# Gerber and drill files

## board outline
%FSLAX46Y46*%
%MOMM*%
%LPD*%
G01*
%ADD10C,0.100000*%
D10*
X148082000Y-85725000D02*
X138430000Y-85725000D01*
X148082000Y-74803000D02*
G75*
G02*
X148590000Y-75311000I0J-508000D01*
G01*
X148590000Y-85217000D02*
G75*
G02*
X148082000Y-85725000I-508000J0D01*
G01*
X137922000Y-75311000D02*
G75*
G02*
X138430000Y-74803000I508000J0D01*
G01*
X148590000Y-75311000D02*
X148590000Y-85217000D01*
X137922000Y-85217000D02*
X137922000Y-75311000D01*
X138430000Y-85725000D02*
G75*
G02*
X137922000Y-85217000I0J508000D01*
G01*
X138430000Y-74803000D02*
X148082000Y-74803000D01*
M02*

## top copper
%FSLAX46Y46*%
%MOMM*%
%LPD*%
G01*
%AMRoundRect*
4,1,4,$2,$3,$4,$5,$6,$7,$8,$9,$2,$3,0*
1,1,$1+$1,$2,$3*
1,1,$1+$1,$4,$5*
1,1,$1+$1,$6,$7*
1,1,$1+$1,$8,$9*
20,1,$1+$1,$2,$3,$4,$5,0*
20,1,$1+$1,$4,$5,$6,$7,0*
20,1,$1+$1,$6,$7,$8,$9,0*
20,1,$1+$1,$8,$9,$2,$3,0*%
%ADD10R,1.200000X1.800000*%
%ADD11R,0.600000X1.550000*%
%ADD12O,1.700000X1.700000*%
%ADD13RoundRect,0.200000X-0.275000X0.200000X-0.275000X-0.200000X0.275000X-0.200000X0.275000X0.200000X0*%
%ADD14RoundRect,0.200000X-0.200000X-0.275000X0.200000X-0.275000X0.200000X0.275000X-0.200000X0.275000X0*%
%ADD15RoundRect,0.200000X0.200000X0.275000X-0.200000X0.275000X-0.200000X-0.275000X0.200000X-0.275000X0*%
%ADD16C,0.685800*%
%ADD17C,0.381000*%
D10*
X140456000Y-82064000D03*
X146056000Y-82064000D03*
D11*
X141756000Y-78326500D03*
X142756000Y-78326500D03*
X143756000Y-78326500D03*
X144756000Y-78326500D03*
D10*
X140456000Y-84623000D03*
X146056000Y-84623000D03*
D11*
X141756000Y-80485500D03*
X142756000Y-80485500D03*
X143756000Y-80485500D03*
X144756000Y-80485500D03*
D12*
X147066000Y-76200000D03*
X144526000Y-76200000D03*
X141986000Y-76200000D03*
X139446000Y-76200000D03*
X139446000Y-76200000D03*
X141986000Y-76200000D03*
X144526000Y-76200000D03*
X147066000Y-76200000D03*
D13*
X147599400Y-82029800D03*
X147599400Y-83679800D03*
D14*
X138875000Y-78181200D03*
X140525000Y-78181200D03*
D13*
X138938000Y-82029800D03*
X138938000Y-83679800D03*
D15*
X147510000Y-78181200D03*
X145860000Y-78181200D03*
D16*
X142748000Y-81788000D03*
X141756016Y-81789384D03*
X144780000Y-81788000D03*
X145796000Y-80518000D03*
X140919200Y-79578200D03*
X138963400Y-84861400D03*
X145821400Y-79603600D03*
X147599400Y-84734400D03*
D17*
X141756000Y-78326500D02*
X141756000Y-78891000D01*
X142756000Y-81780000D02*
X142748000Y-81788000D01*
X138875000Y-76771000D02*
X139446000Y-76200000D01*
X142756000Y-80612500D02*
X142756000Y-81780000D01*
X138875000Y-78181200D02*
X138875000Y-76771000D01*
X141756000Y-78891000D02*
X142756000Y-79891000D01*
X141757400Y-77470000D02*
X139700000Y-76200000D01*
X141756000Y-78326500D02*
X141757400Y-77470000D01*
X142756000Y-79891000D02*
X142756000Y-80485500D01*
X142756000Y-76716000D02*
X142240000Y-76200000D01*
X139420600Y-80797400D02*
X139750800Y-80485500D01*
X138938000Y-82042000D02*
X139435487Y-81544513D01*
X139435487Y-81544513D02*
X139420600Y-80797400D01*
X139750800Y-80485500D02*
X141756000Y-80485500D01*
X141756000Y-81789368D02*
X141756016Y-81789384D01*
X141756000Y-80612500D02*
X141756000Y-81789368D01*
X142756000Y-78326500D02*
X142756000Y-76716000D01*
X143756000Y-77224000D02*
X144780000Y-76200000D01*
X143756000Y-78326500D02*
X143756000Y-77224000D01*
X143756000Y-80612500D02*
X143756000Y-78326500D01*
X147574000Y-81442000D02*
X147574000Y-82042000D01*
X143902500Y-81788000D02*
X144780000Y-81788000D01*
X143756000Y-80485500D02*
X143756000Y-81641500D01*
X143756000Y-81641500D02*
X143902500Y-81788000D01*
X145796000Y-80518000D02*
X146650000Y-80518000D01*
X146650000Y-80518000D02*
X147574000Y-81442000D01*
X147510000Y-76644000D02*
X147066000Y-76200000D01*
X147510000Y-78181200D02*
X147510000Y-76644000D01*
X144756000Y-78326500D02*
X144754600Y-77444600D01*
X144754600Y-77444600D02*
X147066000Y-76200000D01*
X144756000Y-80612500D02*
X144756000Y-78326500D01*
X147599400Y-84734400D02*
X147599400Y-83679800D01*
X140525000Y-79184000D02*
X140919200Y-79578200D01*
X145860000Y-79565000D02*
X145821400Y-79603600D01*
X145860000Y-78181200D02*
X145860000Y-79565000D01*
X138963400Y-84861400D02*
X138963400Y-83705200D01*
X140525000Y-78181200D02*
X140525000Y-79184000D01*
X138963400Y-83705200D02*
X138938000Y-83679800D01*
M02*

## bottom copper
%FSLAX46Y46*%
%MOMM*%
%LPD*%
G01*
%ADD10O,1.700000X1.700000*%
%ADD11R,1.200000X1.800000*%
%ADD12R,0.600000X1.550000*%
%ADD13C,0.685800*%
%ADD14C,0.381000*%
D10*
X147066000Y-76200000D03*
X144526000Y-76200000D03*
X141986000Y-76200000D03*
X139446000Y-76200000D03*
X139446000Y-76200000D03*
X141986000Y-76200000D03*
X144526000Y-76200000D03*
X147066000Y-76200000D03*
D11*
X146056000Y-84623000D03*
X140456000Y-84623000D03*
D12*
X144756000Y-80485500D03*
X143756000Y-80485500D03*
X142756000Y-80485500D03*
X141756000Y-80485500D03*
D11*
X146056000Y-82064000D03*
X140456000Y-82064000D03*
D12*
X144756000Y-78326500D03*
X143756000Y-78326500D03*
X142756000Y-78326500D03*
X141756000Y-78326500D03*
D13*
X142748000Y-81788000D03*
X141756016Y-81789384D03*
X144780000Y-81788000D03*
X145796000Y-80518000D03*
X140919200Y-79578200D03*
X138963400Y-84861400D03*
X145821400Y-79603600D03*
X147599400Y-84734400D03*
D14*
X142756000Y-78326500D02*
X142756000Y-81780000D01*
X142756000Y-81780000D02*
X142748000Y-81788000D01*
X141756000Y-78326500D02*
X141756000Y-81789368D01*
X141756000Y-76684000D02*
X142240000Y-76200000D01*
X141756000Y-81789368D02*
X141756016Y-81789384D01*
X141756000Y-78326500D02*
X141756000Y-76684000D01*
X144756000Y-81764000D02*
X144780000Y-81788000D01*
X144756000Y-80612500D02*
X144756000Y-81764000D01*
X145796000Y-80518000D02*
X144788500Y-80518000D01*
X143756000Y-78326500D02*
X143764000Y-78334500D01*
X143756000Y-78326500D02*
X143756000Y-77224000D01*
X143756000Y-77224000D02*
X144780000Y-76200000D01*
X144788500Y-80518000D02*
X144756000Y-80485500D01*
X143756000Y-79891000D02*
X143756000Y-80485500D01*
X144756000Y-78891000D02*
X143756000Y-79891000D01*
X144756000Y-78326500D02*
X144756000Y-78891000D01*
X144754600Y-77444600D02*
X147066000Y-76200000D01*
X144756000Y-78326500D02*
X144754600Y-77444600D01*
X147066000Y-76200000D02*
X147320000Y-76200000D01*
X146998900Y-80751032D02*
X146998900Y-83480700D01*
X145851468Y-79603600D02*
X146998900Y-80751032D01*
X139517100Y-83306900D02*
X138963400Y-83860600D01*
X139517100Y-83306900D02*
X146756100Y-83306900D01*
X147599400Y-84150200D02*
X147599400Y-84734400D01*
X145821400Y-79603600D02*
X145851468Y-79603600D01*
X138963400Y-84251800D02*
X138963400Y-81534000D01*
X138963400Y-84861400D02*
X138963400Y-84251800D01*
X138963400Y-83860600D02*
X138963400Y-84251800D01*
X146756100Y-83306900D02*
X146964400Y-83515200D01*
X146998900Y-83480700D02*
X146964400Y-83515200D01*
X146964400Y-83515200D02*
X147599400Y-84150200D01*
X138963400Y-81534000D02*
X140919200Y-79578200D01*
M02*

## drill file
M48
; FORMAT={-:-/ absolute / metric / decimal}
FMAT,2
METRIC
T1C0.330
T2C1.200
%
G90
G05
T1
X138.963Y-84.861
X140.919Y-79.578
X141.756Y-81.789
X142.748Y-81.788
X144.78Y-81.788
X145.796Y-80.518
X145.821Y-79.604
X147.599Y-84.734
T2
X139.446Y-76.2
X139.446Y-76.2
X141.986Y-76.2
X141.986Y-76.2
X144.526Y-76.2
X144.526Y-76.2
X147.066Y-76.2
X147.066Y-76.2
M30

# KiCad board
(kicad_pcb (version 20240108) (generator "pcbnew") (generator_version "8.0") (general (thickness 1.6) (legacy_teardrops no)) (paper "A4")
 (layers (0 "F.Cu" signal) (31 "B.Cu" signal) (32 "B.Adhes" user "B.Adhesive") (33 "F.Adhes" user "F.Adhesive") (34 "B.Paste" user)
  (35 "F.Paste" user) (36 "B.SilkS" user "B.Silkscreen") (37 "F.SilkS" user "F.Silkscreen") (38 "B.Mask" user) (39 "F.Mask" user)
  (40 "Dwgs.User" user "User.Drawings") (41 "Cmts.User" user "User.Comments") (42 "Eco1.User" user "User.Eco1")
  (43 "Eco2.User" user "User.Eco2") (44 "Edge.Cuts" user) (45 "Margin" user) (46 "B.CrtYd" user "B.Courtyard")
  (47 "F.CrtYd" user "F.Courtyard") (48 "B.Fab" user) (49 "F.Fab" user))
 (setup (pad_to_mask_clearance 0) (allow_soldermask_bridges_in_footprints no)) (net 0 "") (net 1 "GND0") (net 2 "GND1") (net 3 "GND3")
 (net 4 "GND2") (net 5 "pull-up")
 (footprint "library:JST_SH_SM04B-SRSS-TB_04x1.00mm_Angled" (layer "F.Cu") (at 143.256 80.264)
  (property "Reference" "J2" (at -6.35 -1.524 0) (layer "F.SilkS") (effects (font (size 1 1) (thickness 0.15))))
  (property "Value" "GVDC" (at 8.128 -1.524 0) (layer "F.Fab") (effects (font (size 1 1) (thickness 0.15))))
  (pad "" smd rect (at -2.8 1.8) (size 1.2 1.8) (layers "F.Cu" "F.Paste" "F.Mask"))
  (pad "" smd rect (at 2.8 1.8) (size 1.2 1.8) (layers "F.Cu" "F.Paste" "F.Mask"))
  (pad "1" smd rect (at -1.5 -1.9375) (size 0.6 1.55) (layers "F.Cu" "F.Paste" "F.Mask") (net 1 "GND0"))
  (pad "2" smd rect (at -0.5 -1.9375) (size 0.6 1.55) (layers "F.Cu" "F.Paste" "F.Mask") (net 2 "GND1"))
  (pad "3" smd rect (at 0.5 -1.9375) (size 0.6 1.55) (layers "F.Cu" "F.Paste" "F.Mask") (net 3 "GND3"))
  (pad "4" smd rect (at 1.5 -1.9375) (size 0.6 1.55) (layers "F.Cu" "F.Paste" "F.Mask") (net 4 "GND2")))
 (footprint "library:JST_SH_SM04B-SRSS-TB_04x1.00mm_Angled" (layer "F.Cu") (at 143.256 82.423)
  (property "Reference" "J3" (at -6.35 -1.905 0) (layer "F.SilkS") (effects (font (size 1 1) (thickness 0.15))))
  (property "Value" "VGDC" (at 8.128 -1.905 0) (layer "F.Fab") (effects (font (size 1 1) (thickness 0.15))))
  (pad "" smd rect (at -2.8 2.2) (size 1.2 1.8) (layers "F.Cu" "F.Paste" "F.Mask"))
  (pad "" smd rect (at 2.8 2.2) (size 1.2 1.8) (layers "F.Cu" "F.Paste" "F.Mask"))
  (pad "1" smd rect (at -1.5 -1.9375) (size 0.6 1.55) (layers "F.Cu" "F.Paste" "F.Mask") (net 2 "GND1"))
  (pad "2" smd rect (at -0.5 -1.9375) (size 0.6 1.55) (layers "F.Cu" "F.Paste" "F.Mask") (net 1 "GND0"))
  (pad "3" smd rect (at 0.5 -1.9375) (size 0.6 1.55) (layers "F.Cu" "F.Paste" "F.Mask") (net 3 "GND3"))
  (pad "4" smd rect (at 1.5 -1.9375) (size 0.6 1.55) (layers "F.Cu" "F.Paste" "F.Mask") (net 4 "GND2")))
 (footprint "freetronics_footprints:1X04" (layer "F.Cu") (at 147.066 76.2 180)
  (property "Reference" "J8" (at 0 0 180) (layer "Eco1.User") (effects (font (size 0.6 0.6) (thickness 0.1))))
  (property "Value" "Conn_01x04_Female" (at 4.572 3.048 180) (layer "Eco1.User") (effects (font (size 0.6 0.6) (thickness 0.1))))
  (pad "1" thru_hole oval (at 0 0 270) (size 1.7 1.7) (drill 1.2) (layers "*.Cu" "*.Mask") (remove_unused_layers no) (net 4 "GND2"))
  (pad "2" thru_hole oval (at 2.54 0 270) (size 1.7 1.7) (drill 1.2) (layers "*.Cu" "*.Mask") (remove_unused_layers no) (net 3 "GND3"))
  (pad "3" thru_hole oval (at 5.08 0 270) (size 1.7 1.7) (drill 1.2) (layers "*.Cu" "*.Mask") (remove_unused_layers no) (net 2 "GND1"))
  (pad "4" thru_hole oval (at 7.62 0 270) (size 1.7 1.7) (drill 1.2) (layers "*.Cu" "*.Mask") (remove_unused_layers no) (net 1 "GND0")))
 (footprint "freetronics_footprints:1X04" (layer "F.Cu") (at 139.446 76.2)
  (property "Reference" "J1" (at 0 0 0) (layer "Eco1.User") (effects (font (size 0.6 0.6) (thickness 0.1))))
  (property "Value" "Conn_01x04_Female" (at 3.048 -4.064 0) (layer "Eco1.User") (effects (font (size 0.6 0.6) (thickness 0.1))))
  (pad "1" thru_hole oval (at 0 0 90) (size 1.7 1.7) (drill 1.2) (layers "*.Cu" "*.Mask") (remove_unused_layers no) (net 1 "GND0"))
  (pad "2" thru_hole oval (at 2.54 0 90) (size 1.7 1.7) (drill 1.2) (layers "*.Cu" "*.Mask") (remove_unused_layers no) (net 2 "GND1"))
  (pad "3" thru_hole oval (at 5.08 0 90) (size 1.7 1.7) (drill 1.2) (layers "*.Cu" "*.Mask") (remove_unused_layers no) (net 3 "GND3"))
  (pad "4" thru_hole oval (at 7.62 0 90) (size 1.7 1.7) (drill 1.2) (layers "*.Cu" "*.Mask") (remove_unused_layers no) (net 4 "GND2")))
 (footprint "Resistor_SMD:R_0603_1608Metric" (layer "F.Cu") (at 147.5994 82.8548 -90)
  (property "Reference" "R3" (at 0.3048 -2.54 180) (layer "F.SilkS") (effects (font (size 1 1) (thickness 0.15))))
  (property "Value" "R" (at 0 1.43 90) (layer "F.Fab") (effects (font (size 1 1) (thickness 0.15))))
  (pad "1" smd roundrect (at -0.825 0 270) (size 0.8 0.95) (layers "F.Cu" "F.Paste" "F.Mask") (roundrect_rratio 0.25) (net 3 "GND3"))
  (pad "2" smd roundrect (at 0.825 0 270) (size 0.8 0.95) (layers "F.Cu" "F.Paste" "F.Mask") (roundrect_rratio 0.25) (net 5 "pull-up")))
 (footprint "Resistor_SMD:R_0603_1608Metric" (layer "F.Cu") (at 139.7 78.1812)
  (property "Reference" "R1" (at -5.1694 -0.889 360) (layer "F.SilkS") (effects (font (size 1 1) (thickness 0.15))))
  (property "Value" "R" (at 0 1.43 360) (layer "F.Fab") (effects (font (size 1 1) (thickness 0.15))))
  (pad "1" smd roundrect (at -0.825 0) (size 0.8 0.95) (layers "F.Cu" "F.Paste" "F.Mask") (roundrect_rratio 0.25) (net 1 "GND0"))
  (pad "2" smd roundrect (at 0.825 0) (size 0.8 0.95) (layers "F.Cu" "F.Paste" "F.Mask") (roundrect_rratio 0.25) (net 5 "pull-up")))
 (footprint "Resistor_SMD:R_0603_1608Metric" (layer "F.Cu") (at 138.938 82.8548 -90)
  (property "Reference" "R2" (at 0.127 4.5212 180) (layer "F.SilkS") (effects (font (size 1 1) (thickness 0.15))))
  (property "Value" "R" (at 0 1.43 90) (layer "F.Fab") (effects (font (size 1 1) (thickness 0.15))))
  (pad "1" smd roundrect (at -0.825 0 270) (size 0.8 0.95) (layers "F.Cu" "F.Paste" "F.Mask") (roundrect_rratio 0.25) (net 2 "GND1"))
  (pad "2" smd roundrect (at 0.825 0 270) (size 0.8 0.95) (layers "F.Cu" "F.Paste" "F.Mask") (roundrect_rratio 0.25) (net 5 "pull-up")))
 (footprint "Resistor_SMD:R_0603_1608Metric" (layer "F.Cu") (at 146.685 78.1812 180)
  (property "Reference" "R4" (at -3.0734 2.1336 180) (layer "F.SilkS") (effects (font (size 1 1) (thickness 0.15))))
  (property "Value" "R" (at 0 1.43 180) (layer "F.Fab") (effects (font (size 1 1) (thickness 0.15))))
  (pad "1" smd roundrect (at -0.825 0 180) (size 0.8 0.95) (layers "F.Cu" "F.Paste" "F.Mask") (roundrect_rratio 0.25) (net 4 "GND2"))
  (pad "2" smd roundrect (at 0.825 0 180) (size 0.8 0.95) (layers "F.Cu" "F.Paste" "F.Mask") (roundrect_rratio 0.25) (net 5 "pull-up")))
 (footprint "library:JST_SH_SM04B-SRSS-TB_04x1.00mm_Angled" (layer "B.Cu") (at 143.256 82.423 180)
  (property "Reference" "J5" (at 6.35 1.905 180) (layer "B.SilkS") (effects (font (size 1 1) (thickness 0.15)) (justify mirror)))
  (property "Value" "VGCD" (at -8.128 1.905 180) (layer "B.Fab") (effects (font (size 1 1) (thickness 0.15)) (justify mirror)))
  (pad "" smd rect (at -2.8 -2.2 180) (size 1.2 1.8) (layers "B.Cu" "B.Paste" "B.Mask"))
  (pad "" smd rect (at 2.8 -2.2 180) (size 1.2 1.8) (layers "B.Cu" "B.Paste" "B.Mask"))
  (pad "1" smd rect (at -1.5 1.9375 180) (size 0.6 1.55) (layers "B.Cu" "B.Paste" "B.Mask") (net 3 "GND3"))
  (pad "2" smd rect (at -0.5 1.9375 180) (size 0.6 1.55) (layers "B.Cu" "B.Paste" "B.Mask") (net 4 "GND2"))
  (pad "3" smd rect (at 0.5 1.9375 180) (size 0.6 1.55) (layers "B.Cu" "B.Paste" "B.Mask") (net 1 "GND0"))
  (pad "4" smd rect (at 1.5 1.9375 180) (size 0.6 1.55) (layers "B.Cu" "B.Paste" "B.Mask") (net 2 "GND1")))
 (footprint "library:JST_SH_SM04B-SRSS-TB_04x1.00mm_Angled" (layer "B.Cu") (at 143.256 80.264 180)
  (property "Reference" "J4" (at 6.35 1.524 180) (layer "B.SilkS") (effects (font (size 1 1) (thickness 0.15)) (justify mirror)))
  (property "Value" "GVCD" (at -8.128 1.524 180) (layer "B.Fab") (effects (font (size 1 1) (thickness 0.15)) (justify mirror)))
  (pad "" smd rect (at -2.8 -1.8 180) (size 1.2 1.8) (layers "B.Cu" "B.Paste" "B.Mask"))
  (pad "" smd rect (at 2.8 -1.8 180) (size 1.2 1.8) (layers "B.Cu" "B.Paste" "B.Mask"))
  (pad "1" smd rect (at -1.5 1.9375 180) (size 0.6 1.55) (layers "B.Cu" "B.Paste" "B.Mask") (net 4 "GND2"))
  (pad "2" smd rect (at -0.5 1.9375 180) (size 0.6 1.55) (layers "B.Cu" "B.Paste" "B.Mask") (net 3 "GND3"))
  (pad "3" smd rect (at 0.5 1.9375 180) (size 0.6 1.55) (layers "B.Cu" "B.Paste" "B.Mask") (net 1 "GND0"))
  (pad "4" smd rect (at 1.5 1.9375 180) (size 0.6 1.55) (layers "B.Cu" "B.Paste" "B.Mask") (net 2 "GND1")))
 (gr_line (start 148.082 85.725) (end 138.43 85.725) (stroke (width 0.1) (type solid)) (layer "Edge.Cuts"))
 (gr_arc (start 148.082 74.803) (mid 148.44121 74.95179) (end 148.59 75.311) (stroke (width 0.1) (type solid)) (layer "Edge.Cuts"))
 (gr_arc (start 148.59 85.217) (mid 148.44121 85.57621) (end 148.082 85.725) (stroke (width 0.1) (type solid)) (layer "Edge.Cuts"))
 (gr_arc (start 137.922 75.311) (mid 138.07079 74.95179) (end 138.43 74.803) (stroke (width 0.1) (type solid)) (layer "Edge.Cuts"))
 (gr_line (start 148.59 75.311) (end 148.59 85.217) (stroke (width 0.1) (type solid)) (layer "Edge.Cuts"))
 (gr_line (start 137.922 85.217) (end 137.922 75.311) (stroke (width 0.1) (type solid)) (layer "Edge.Cuts"))
 (gr_arc (start 138.43 85.725) (mid 138.07079 85.57621) (end 137.922 85.217) (stroke (width 0.1) (type solid)) (layer "Edge.Cuts"))
 (gr_line (start 138.43 74.803) (end 148.082 74.803) (stroke (width 0.1) (type solid)) (layer "Edge.Cuts"))
 (segment (start 141.756 78.3265) (end 141.756 78.891) (width 0.381) (layer "F.Cu") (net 1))
 (segment (start 142.756 81.78) (end 142.748 81.788) (width 0.381) (layer "F.Cu") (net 1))
 (segment (start 138.875 76.771) (end 139.446 76.2) (width 0.381) (layer "F.Cu") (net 1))
 (segment (start 142.756 80.6125) (end 142.756 81.78) (width 0.381) (layer "F.Cu") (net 1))
 (segment (start 138.875 78.1812) (end 138.875 76.771) (width 0.381) (layer "F.Cu") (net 1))
 (segment (start 141.756 78.891) (end 142.756 79.891) (width 0.381) (layer "F.Cu") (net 1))
 (segment (start 141.7574 77.47) (end 139.7 76.2) (width 0.381) (layer "F.Cu") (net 1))
 (segment (start 141.756 78.3265) (end 141.7574 77.47) (width 0.381) (layer "F.Cu") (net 1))
 (segment (start 142.756 79.891) (end 142.756 80.4855) (width 0.381) (layer "F.Cu") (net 1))
 (via (at 142.748 81.788) (size 0.6858) (drill 0.3302) (layers "F.Cu" "B.Cu") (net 1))
 (segment (start 142.756 78.3265) (end 142.756 81.78) (width 0.381) (layer "B.Cu") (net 1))
 (segment (start 142.756 81.78) (end 142.748 81.788) (width 0.381) (layer "B.Cu") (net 1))
 (segment (start 142.756 76.716) (end 142.24 76.2) (width 0.381) (layer "F.Cu") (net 2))
 (segment (start 139.4206 80.7974) (end 139.7508 80.4855) (width 0.381) (layer "F.Cu") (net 2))
 (segment (start 138.938 82.042) (end 139.435487 81.544513) (width 0.381) (layer "F.Cu") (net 2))
 (segment (start 139.435487 81.544513) (end 139.4206 80.7974) (width 0.381) (layer "F.Cu") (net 2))
 (segment (start 139.7508 80.4855) (end 141.756 80.4855) (width 0.381) (layer "F.Cu") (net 2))
 (segment (start 141.756 81.789368) (end 141.756016 81.789384) (width 0.381) (layer "F.Cu") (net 2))
 (segment (start 141.756 80.6125) (end 141.756 81.789368) (width 0.381) (layer "F.Cu") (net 2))
 (segment (start 142.756 78.3265) (end 142.756 76.716) (width 0.381) (layer "F.Cu") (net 2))
 (via (at 141.756016 81.789384) (size 0.6858) (drill 0.3302) (layers "F.Cu" "B.Cu") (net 2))
 (segment (start 141.756 78.3265) (end 141.756 81.789368) (width 0.381) (layer "B.Cu") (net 2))
 (segment (start 141.756 76.684) (end 142.24 76.2) (width 0.381) (layer "B.Cu") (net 2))
 (segment (start 141.756 81.789368) (end 141.756016 81.789384) (width 0.381) (layer "B.Cu") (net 2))
 (segment (start 141.756 78.3265) (end 141.756 76.684) (width 0.381) (layer "B.Cu") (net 2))
 (segment (start 143.756 77.224) (end 144.78 76.2) (width 0.381) (layer "F.Cu") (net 3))
 (segment (start 143.756 78.3265) (end 143.756 77.224) (width 0.381) (layer "F.Cu") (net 3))
 (segment (start 143.756 80.6125) (end 143.756 78.3265) (width 0.381) (layer "F.Cu") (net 3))
 (segment (start 147.574 81.442) (end 147.574 82.042) (width 0.381) (layer "F.Cu") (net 3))
 (segment (start 143.9025 81.788) (end 144.78 81.788) (width 0.381) (layer "F.Cu") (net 3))
 (segment (start 143.756 80.4855) (end 143.756 81.6415) (width 0.381) (layer "F.Cu") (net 3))
 (segment (start 143.756 81.6415) (end 143.9025 81.788) (width 0.381) (layer "F.Cu") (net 3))
 (segment (start 145.796 80.518) (end 146.65 80.518) (width 0.381) (layer "F.Cu") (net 3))
 (segment (start 146.65 80.518) (end 147.574 81.442) (width 0.381) (layer "F.Cu") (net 3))
 (via (at 144.78 81.788) (size 0.6858) (drill 0.3302) (layers "F.Cu" "B.Cu") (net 3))
 (via (at 145.796 80.518) (size 0.6858) (drill 0.3302) (layers "F.Cu" "B.Cu") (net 3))
 (segment (start 144.756 81.764) (end 144.78 81.788) (width 0.381) (layer "B.Cu") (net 3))
 (segment (start 144.756 80.6125) (end 144.756 81.764) (width 0.381) (layer "B.Cu") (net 3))
 (segment (start 145.796 80.518) (end 144.7885 80.518) (width 0.381) (layer "B.Cu") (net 3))
 (segment (start 143.756 78.3265) (end 143.764 78.3345) (width 0.381) (layer "B.Cu") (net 3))
 (segment (start 143.756 78.3265) (end 143.756 77.224) (width 0.381) (layer "B.Cu") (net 3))
 (segment (start 143.756 77.224) (end 144.78 76.2) (width 0.381) (layer "B.Cu") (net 3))
 (segment (start 144.7885 80.518) (end 144.756 80.4855) (width 0.381) (layer "B.Cu") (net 3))
 (segment (start 147.51 76.644) (end 147.066 76.2) (width 0.381) (layer "F.Cu") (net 4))
 (segment (start 147.51 78.1812) (end 147.51 76.644) (width 0.381) (layer "F.Cu") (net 4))
 (segment (start 144.756 78.3265) (end 144.7546 77.4446) (width 0.381) (layer "F.Cu") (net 4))
 (segment (start 144.7546 77.4446) (end 147.066 76.2) (width 0.381) (layer "F.Cu") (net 4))
 (segment (start 144.756 80.6125) (end 144.756 78.3265) (width 0.381) (layer "F.Cu") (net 4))
 (segment (start 143.756 79.891) (end 143.756 80.4855) (width 0.381) (layer "B.Cu") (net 4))
 (segment (start 144.756 78.891) (end 143.756 79.891) (width 0.381) (layer "B.Cu") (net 4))
 (segment (start 144.756 78.3265) (end 144.756 78.891) (width 0.381) (layer "B.Cu") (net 4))
 (segment (start 144.7546 77.4446) (end 147.066 76.2) (width 0.381) (layer "B.Cu") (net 4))
 (segment (start 144.756 78.3265) (end 144.7546 77.4446) (width 0.381) (layer "B.Cu") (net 4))
 (segment (start 147.066 76.2) (end 147.32 76.2) (width 0.381) (layer "B.Cu") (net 4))
 (segment (start 147.5994 84.7344) (end 147.5994 83.6798) (width 0.381) (layer "F.Cu") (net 5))
 (segment (start 140.525 79.184) (end 140.9192 79.5782) (width 0.381) (layer "F.Cu") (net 5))
 (segment (start 145.86 79.565) (end 145.8214 79.6036) (width 0.381) (layer "F.Cu") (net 5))
 (segment (start 145.86 78.1812) (end 145.86 79.565) (width 0.381) (layer "F.Cu") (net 5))
 (segment (start 138.9634 84.8614) (end 138.9634 83.7052) (width 0.381) (layer "F.Cu") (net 5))
 (segment (start 140.525 78.1812) (end 140.525 79.184) (width 0.381) (layer "F.Cu") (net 5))
 (segment (start 138.9634 83.7052) (end 138.938 83.6798) (width 0.381) (layer "F.Cu") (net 5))
 (via (at 140.9192 79.5782) (size 0.6858) (drill 0.3302) (layers "F.Cu" "B.Cu") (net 5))
 (via (at 138.9634 84.8614) (size 0.6858) (drill 0.3302) (layers "F.Cu" "B.Cu") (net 5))
 (via (at 145.8214 79.6036) (size 0.6858) (drill 0.3302) (layers "F.Cu" "B.Cu") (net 5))
 (via (at 147.5994 84.7344) (size 0.6858) (drill 0.3302) (layers "F.Cu" "B.Cu") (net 5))
 (segment (start 146.9989 80.751032) (end 146.9989 83.4807) (width 0.381) (layer "B.Cu") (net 5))
 (segment (start 145.851468 79.6036) (end 146.9989 80.751032) (width 0.381) (layer "B.Cu") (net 5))
 (segment (start 139.5171 83.3069) (end 138.9634 83.8606) (width 0.381) (layer "B.Cu") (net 5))
 (segment (start 139.5171 83.3069) (end 146.7561 83.3069) (width 0.381) (layer "B.Cu") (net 5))
 (segment (start 147.5994 84.1502) (end 147.5994 84.7344) (width 0.381) (layer "B.Cu") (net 5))
 (segment (start 145.8214 79.6036) (end 145.851468 79.6036) (width 0.381) (layer "B.Cu") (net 5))
 (segment (start 138.9634 84.2518) (end 138.9634 81.534) (width 0.381) (layer "B.Cu") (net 5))
 (segment (start 138.9634 84.8614) (end 138.9634 84.2518) (width 0.381) (layer "B.Cu") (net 5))
 (segment (start 138.9634 83.8606) (end 138.9634 84.2518) (width 0.381) (layer "B.Cu") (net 5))
 (segment (start 146.7561 83.3069) (end 146.9644 83.5152) (width 0.381) (layer "B.Cu") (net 5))
 (segment (start 146.9989 83.4807) (end 146.9644 83.5152) (width 0.381) (layer "B.Cu") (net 5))
 (segment (start 146.9644 83.5152) (end 147.5994 84.1502) (width 0.381) (layer "B.Cu") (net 5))
 (segment (start 138.9634 81.534) (end 140.9192 79.5782) (width 0.381) (layer "B.Cu") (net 5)))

